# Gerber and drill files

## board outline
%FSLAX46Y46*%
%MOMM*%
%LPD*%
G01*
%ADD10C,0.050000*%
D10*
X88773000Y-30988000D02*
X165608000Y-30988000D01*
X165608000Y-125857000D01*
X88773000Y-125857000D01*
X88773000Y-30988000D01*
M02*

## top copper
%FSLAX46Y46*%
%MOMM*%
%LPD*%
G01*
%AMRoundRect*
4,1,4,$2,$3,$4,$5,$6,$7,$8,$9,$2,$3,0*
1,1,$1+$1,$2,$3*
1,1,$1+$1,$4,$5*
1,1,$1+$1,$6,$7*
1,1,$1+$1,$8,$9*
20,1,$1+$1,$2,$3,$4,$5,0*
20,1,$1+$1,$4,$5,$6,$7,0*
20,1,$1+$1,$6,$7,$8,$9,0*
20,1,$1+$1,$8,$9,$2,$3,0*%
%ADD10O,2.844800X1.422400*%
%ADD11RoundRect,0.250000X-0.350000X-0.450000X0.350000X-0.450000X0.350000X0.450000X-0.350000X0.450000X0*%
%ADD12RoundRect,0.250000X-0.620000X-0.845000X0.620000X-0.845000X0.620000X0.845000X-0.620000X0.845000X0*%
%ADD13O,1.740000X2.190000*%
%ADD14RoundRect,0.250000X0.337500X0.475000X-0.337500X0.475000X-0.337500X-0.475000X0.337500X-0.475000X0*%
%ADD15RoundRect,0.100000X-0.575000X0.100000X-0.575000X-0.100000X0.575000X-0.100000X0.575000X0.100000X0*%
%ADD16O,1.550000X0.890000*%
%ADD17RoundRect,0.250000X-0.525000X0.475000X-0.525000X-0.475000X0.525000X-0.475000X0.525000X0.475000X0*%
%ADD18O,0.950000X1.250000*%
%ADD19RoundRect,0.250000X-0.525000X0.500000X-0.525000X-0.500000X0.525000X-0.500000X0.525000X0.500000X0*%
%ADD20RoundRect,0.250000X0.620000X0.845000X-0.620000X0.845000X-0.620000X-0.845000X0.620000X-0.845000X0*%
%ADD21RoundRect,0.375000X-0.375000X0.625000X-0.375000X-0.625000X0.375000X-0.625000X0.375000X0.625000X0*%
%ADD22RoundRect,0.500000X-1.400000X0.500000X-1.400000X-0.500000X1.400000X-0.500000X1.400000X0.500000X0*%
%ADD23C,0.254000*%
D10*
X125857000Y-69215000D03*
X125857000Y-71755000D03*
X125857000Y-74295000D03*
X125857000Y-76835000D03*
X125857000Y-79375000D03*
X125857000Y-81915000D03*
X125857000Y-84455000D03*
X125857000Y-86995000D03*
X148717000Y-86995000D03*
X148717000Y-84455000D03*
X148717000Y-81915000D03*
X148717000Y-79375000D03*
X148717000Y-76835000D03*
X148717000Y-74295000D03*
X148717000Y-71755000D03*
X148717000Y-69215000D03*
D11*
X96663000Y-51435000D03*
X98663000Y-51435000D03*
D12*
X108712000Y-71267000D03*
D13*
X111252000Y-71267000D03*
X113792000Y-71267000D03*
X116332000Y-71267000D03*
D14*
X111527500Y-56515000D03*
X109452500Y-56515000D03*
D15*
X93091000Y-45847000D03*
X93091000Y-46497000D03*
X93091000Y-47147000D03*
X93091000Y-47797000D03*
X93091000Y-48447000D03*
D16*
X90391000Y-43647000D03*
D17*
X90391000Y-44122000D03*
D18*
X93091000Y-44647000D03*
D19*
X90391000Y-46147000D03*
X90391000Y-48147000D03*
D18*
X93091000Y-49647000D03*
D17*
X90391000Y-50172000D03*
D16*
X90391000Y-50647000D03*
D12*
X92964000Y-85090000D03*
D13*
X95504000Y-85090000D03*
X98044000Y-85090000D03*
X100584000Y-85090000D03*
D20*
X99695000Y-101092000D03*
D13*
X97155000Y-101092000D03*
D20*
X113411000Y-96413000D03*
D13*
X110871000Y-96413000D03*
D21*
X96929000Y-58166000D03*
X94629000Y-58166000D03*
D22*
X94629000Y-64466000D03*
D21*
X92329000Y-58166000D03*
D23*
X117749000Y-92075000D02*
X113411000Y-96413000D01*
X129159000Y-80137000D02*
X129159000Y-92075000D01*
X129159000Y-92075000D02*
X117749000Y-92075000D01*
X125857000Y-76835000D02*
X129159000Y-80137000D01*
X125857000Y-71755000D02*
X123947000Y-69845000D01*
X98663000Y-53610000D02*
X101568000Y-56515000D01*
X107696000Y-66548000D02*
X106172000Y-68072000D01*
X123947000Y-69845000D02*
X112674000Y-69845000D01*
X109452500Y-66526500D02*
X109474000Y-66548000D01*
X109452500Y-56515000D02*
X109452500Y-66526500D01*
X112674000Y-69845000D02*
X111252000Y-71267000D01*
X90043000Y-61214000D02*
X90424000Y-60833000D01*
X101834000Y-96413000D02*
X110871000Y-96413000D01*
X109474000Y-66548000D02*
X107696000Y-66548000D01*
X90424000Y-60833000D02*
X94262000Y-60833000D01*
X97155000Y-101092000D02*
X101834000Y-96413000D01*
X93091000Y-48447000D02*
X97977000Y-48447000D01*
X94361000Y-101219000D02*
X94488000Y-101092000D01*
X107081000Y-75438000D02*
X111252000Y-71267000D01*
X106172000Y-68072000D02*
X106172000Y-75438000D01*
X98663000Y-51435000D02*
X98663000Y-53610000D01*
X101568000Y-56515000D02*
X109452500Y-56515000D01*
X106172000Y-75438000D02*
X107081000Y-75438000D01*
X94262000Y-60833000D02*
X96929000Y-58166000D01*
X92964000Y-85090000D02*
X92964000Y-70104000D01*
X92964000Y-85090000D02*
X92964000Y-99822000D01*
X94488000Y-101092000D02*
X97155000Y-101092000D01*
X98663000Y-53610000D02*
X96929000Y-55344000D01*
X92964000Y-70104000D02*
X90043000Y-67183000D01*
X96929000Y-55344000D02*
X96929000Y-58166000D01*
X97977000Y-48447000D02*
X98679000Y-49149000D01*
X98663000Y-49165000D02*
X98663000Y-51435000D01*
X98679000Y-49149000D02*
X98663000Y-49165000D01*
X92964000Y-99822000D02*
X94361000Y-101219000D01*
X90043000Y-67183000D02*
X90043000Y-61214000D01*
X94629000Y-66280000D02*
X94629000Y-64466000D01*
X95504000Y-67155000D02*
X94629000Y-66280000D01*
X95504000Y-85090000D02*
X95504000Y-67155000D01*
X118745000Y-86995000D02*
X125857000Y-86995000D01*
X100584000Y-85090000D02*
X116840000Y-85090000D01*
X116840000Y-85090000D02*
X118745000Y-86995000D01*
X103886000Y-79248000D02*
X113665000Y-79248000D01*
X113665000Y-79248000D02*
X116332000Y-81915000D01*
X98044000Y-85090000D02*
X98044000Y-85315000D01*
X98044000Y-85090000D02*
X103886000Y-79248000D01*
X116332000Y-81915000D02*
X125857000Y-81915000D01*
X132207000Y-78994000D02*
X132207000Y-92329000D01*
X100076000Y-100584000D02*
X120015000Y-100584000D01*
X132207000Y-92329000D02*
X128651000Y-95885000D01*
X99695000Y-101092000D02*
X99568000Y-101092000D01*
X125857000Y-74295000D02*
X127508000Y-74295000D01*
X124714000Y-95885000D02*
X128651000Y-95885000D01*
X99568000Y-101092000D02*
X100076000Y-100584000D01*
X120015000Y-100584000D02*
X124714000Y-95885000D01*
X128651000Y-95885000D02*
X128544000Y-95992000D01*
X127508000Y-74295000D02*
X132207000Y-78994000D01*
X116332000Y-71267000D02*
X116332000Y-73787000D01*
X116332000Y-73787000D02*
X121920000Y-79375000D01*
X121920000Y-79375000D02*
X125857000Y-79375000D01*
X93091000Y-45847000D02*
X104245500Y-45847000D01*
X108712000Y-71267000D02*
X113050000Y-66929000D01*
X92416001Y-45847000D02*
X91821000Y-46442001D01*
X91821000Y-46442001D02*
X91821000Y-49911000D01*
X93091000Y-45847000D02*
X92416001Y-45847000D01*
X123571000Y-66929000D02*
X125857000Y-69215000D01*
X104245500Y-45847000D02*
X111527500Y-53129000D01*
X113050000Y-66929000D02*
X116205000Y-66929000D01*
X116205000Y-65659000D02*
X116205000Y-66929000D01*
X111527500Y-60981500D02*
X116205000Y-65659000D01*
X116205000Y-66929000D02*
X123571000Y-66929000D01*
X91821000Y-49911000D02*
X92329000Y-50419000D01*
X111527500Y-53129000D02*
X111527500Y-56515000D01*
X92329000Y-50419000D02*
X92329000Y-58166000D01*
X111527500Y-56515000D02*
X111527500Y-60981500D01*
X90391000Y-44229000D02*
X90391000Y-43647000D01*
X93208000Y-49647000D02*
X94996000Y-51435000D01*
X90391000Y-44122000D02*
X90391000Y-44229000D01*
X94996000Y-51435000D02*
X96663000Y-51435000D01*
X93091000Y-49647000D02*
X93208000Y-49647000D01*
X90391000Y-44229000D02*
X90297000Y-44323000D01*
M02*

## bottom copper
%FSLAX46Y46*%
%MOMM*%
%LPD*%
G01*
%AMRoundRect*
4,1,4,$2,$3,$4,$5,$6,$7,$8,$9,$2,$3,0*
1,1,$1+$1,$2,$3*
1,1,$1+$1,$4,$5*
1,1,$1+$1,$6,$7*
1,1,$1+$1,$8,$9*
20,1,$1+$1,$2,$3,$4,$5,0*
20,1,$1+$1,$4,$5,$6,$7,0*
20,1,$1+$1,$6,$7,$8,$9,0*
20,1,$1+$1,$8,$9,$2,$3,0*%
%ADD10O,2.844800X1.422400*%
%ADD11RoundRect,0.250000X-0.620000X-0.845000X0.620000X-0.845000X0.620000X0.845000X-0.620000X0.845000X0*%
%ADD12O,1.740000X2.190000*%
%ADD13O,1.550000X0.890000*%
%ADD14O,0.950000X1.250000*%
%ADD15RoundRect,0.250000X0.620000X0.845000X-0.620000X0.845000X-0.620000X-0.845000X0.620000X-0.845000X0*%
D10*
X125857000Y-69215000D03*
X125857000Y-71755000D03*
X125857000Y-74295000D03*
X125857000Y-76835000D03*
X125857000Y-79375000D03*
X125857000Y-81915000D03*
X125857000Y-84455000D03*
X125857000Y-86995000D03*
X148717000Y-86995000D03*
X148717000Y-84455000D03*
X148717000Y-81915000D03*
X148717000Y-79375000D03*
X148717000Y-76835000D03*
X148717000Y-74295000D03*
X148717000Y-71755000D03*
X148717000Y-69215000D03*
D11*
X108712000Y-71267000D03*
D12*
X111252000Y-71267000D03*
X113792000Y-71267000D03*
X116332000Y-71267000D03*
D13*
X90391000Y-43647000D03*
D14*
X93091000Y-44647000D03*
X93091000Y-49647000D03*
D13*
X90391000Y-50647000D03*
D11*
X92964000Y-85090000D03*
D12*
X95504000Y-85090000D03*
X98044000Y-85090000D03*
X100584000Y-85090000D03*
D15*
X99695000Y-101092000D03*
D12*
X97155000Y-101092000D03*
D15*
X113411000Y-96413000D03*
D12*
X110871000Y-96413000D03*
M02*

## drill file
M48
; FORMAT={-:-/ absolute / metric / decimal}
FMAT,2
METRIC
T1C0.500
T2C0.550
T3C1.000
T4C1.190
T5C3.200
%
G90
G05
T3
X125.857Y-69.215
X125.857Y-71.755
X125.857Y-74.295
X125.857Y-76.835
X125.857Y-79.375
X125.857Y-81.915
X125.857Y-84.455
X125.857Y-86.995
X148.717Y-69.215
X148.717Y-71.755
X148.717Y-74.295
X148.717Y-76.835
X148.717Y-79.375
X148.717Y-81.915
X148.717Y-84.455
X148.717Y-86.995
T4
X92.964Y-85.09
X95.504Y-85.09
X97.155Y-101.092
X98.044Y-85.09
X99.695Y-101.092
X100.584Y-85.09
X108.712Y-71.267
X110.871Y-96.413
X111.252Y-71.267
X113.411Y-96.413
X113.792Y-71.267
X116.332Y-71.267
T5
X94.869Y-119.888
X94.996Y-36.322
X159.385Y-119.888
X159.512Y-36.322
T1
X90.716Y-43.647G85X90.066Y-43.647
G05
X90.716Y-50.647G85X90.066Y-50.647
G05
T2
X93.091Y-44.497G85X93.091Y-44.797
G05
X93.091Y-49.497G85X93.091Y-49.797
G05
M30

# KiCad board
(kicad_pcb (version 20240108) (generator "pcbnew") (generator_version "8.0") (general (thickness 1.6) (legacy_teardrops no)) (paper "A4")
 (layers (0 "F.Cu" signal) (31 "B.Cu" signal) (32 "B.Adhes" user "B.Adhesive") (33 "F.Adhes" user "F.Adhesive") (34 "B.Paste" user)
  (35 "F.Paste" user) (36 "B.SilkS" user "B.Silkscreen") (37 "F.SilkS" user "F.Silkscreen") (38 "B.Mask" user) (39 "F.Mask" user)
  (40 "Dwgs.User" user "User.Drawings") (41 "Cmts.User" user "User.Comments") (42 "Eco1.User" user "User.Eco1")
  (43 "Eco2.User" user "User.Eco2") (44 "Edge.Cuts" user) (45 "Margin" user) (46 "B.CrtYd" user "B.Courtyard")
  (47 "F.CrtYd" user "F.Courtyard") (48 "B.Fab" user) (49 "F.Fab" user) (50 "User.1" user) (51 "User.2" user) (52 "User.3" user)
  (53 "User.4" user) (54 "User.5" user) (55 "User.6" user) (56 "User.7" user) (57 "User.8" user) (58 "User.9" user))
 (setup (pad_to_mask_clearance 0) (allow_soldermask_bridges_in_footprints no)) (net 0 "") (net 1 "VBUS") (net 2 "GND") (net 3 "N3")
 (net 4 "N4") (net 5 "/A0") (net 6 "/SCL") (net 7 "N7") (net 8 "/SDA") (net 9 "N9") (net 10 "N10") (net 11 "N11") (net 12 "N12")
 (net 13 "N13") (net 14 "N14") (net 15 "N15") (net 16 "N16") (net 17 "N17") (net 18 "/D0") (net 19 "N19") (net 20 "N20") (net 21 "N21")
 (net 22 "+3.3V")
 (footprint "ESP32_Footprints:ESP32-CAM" (layer "F.Cu") (at 137.287 79.375)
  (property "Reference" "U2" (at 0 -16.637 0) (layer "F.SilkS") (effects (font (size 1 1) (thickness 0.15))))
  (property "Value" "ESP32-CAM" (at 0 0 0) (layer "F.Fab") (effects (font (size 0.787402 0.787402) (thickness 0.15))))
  (pad "P$1" thru_hole oval (at -11.43 -10.16) (size 2.8448 1.4224) (drill 1) (layers "*.Cu" "*.Mask") (remove_unused_layers no)
   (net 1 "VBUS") (solder_mask_margin 0.102))
  (pad "P$2" thru_hole oval (at -11.43 -7.62) (size 2.8448 1.4224) (drill 1) (layers "*.Cu" "*.Mask") (remove_unused_layers no)
   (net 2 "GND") (solder_mask_margin 0.102))
  (pad "P$3" thru_hole oval (at -11.43 -5.08) (size 2.8448 1.4224) (drill 1) (layers "*.Cu" "*.Mask") (remove_unused_layers no) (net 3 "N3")
   (solder_mask_margin 0.102))
  (pad "P$4" thru_hole oval (at -11.43 -2.54) (size 2.8448 1.4224) (drill 1) (layers "*.Cu" "*.Mask") (remove_unused_layers no) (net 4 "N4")
   (solder_mask_margin 0.102))
  (pad "P$5" thru_hole oval (at -11.43 0) (size 2.8448 1.4224) (drill 1) (layers "*.Cu" "*.Mask") (remove_unused_layers no) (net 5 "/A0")
   (solder_mask_margin 0.102))
  (pad "P$6" thru_hole oval (at -11.43 2.54) (size 2.8448 1.4224) (drill 1) (layers "*.Cu" "*.Mask") (remove_unused_layers no)
   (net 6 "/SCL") (solder_mask_margin 0.102))
  (pad "P$7" thru_hole oval (at -11.43 5.08) (size 2.8448 1.4224) (drill 1) (layers "*.Cu" "*.Mask") (remove_unused_layers no) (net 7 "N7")
   (solder_mask_margin 0.102))
  (pad "P$8" thru_hole oval (at -11.43 7.62) (size 2.8448 1.4224) (drill 1) (layers "*.Cu" "*.Mask") (remove_unused_layers no)
   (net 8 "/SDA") (solder_mask_margin 0.102))
  (pad "P$9" thru_hole oval (at 11.43 7.62) (size 2.8448 1.4224) (drill 1) (layers "*.Cu" "*.Mask") (remove_unused_layers no) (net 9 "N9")
   (solder_mask_margin 0.102))
  (pad "P$10" thru_hole oval (at 11.43 5.08) (size 2.8448 1.4224) (drill 1) (layers "*.Cu" "*.Mask") (remove_unused_layers no)
   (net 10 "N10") (solder_mask_margin 0.102))
  (pad "P$11" thru_hole oval (at 11.43 2.54) (size 2.8448 1.4224) (drill 1) (layers "*.Cu" "*.Mask") (remove_unused_layers no)
   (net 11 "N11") (solder_mask_margin 0.102))
  (pad "P$12" thru_hole oval (at 11.43 0) (size 2.8448 1.4224) (drill 1) (layers "*.Cu" "*.Mask") (remove_unused_layers no) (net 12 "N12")
   (solder_mask_margin 0.102))
  (pad "P$13" thru_hole oval (at 11.43 -2.54) (size 2.8448 1.4224) (drill 1) (layers "*.Cu" "*.Mask") (remove_unused_layers no)
   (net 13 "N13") (solder_mask_margin 0.102))
  (pad "P$14" thru_hole oval (at 11.43 -5.08) (size 2.8448 1.4224) (drill 1) (layers "*.Cu" "*.Mask") (remove_unused_layers no)
   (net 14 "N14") (solder_mask_margin 0.102))
  (pad "P$15" thru_hole oval (at 11.43 -7.62) (size 2.8448 1.4224) (drill 1) (layers "*.Cu" "*.Mask") (remove_unused_layers no)
   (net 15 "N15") (solder_mask_margin 0.102))
  (pad "P$16" thru_hole oval (at 11.43 -10.16) (size 2.8448 1.4224) (drill 1) (layers "*.Cu" "*.Mask") (remove_unused_layers no)
   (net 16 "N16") (solder_mask_margin 0.102)))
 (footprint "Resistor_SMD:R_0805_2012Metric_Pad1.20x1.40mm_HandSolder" (layer "F.Cu") (at 97.663 51.435)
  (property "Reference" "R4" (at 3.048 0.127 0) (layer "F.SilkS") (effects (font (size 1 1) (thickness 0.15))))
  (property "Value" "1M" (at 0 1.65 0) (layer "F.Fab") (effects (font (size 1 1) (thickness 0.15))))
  (pad "1" smd roundrect (at -1 0) (size 1.2 1.4) (layers "F.Cu" "F.Paste" "F.Mask") (roundrect_rratio 0.208333) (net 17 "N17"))
  (pad "2" smd roundrect (at 1 0) (size 1.2 1.4) (layers "F.Cu" "F.Paste" "F.Mask") (roundrect_rratio 0.208333) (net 2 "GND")))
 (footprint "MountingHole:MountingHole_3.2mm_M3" (layer "F.Cu") (at 159.512 36.322)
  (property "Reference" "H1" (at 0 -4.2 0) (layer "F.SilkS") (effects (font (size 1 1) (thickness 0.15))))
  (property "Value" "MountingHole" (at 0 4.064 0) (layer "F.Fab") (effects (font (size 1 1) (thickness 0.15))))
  (pad "" np_thru_hole circle (at 0 0) (size 3.2 3.2) (drill 3.2) (layers "*.Cu" "*.Mask")))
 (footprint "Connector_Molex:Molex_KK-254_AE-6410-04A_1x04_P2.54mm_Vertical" (layer "F.Cu") (at 108.712 71.267)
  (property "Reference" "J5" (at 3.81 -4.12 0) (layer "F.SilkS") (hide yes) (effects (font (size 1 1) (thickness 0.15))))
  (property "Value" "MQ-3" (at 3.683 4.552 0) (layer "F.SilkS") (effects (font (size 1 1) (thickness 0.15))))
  (pad "1" thru_hole roundrect (at 0 0) (size 1.74 2.19) (drill 1.19) (layers "*.Cu" "*.Mask") (remove_unused_layers no)
   (roundrect_rratio 0.143678) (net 1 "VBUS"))
  (pad "2" thru_hole oval (at 2.54 0) (size 1.74 2.19) (drill 1.19) (layers "*.Cu" "*.Mask") (remove_unused_layers no) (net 2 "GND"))
  (pad "3" thru_hole oval (at 5.08 0) (size 1.74 2.19) (drill 1.19) (layers "*.Cu" "*.Mask") (remove_unused_layers no) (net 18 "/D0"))
  (pad "4" thru_hole oval (at 7.62 0) (size 1.74 2.19) (drill 1.19) (layers "*.Cu" "*.Mask") (remove_unused_layers no) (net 5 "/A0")))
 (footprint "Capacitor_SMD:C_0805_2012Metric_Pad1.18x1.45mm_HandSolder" (layer "F.Cu") (at 110.49 56.515 180)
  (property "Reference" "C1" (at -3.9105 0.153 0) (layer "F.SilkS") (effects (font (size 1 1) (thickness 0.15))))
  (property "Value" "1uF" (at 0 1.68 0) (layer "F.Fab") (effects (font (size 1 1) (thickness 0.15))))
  (pad "1" smd roundrect (at -1.0375 0 180) (size 1.175 1.45) (layers "F.Cu" "F.Paste" "F.Mask") (roundrect_rratio 0.212766) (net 1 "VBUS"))
  (pad "2" smd roundrect (at 1.0375 0 180) (size 1.175 1.45) (layers "F.Cu" "F.Paste" "F.Mask") (roundrect_rratio 0.212766) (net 2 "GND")))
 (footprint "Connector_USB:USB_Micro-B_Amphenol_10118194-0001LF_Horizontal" (layer "F.Cu") (at 91.691 47.147 -90)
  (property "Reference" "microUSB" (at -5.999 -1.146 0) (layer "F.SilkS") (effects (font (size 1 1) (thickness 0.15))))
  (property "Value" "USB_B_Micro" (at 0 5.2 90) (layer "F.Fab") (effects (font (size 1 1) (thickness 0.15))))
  (pad "" smd oval (at -3.5 1.3 270) (size 0.89 1.55) (layers "F.Paste"))
  (pad "" smd oval (at -2.5 -1.4 270) (size 1.25 0.95) (layers "F.Paste"))
  (pad "" smd oval (at 2.5 -1.4 270) (size 1.25 0.95) (layers "F.Paste"))
  (pad "" smd oval (at 3.5 1.3 270) (size 0.89 1.55) (layers "F.Paste"))
  (pad "1" smd roundrect (at -1.3 -1.4 270) (size 0.4 1.35) (layers "F.Cu" "F.Paste" "F.Mask") (roundrect_rratio 0.25) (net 1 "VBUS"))
  (pad "2" smd roundrect (at -0.65 -1.4 270) (size 0.4 1.35) (layers "F.Cu" "F.Paste" "F.Mask") (roundrect_rratio 0.25) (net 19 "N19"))
  (pad "3" smd roundrect (at 0 -1.4 270) (size 0.4 1.35) (layers "F.Cu" "F.Paste" "F.Mask") (roundrect_rratio 0.25) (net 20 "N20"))
  (pad "4" smd roundrect (at 0.65 -1.4 270) (size 0.4 1.35) (layers "F.Cu" "F.Paste" "F.Mask") (roundrect_rratio 0.25) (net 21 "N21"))
  (pad "5" smd roundrect (at 1.3 -1.4 270) (size 0.4 1.35) (layers "F.Cu" "F.Paste" "F.Mask") (roundrect_rratio 0.25) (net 2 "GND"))
  (pad "6" thru_hole oval (at -3.5 1.3 270) (size 0.89 1.55) (drill oval 0.5 1.15) (layers "*.Cu" "*.Mask") (remove_unused_layers no)
   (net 17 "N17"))
  (pad "6" smd roundrect (at -3.025 1.3 270) (size 1.45 1.55) (layers "F.Cu" "F.Paste" "F.Mask") (roundrect_rratio 0.1724137931)
   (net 17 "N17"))
  (pad "6" thru_hole oval (at -2.5 -1.4 270) (size 1.25 0.95) (drill oval 0.85 0.55) (layers "*.Cu" "*.Mask") (remove_unused_layers no)
   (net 17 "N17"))
  (pad "6" smd roundrect (at -1 1.3 270) (size 1.5 1.55) (layers "F.Cu" "F.Paste" "F.Mask") (roundrect_rratio 0.1666666667) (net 17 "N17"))
  (pad "6" smd roundrect (at 1 1.3 270) (size 1.5 1.55) (layers "F.Cu" "F.Paste" "F.Mask") (roundrect_rratio 0.1666666667) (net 17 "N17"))
  (pad "6" thru_hole oval (at 2.5 -1.4 270) (size 1.25 0.95) (drill oval 0.85 0.55) (layers "*.Cu" "*.Mask") (remove_unused_layers no)
   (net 17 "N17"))
  (pad "6" smd roundrect (at 3.025 1.3 270) (size 1.45 1.55) (layers "F.Cu" "F.Paste" "F.Mask") (roundrect_rratio 0.1724137931)
   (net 17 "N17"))
  (pad "6" thru_hole oval (at 3.5 1.3 270) (size 0.89 1.55) (drill oval 0.5 1.15) (layers "*.Cu" "*.Mask") (remove_unused_layers no)
   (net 17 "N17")))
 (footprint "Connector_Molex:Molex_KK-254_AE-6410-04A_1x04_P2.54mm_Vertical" (layer "F.Cu") (at 92.964 85.09)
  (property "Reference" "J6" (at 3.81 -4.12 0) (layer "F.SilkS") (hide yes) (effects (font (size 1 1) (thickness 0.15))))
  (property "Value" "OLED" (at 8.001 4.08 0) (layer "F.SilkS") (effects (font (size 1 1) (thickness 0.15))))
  (pad "1" thru_hole roundrect (at 0 0) (size 1.74 2.19) (drill 1.19) (layers "*.Cu" "*.Mask") (remove_unused_layers no)
   (roundrect_rratio 0.143678) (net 2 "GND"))
  (pad "2" thru_hole oval (at 2.54 0) (size 1.74 2.19) (drill 1.19) (layers "*.Cu" "*.Mask") (remove_unused_layers no) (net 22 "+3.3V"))
  (pad "3" thru_hole oval (at 5.08 0) (size 1.74 2.19) (drill 1.19) (layers "*.Cu" "*.Mask") (remove_unused_layers no) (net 6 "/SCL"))
  (pad "4" thru_hole oval (at 7.62 0) (size 1.74 2.19) (drill 1.19) (layers "*.Cu" "*.Mask") (remove_unused_layers no) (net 8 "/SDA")))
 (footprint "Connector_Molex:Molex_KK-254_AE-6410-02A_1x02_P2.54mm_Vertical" (layer "F.Cu") (at 99.695 101.092 180)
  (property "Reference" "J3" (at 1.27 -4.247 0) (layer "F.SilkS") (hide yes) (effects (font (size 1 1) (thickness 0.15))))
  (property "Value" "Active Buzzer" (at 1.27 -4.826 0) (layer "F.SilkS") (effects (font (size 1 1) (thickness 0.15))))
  (pad "1" thru_hole roundrect (at 0 0 180) (size 1.74 2.19) (drill 1.19) (layers "*.Cu" "*.Mask") (remove_unused_layers no)
   (roundrect_rratio 0.143678) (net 3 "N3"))
  (pad "2" thru_hole oval (at 2.54 0 180) (size 1.74 2.19) (drill 1.19) (layers "*.Cu" "*.Mask") (remove_unused_layers no) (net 2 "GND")))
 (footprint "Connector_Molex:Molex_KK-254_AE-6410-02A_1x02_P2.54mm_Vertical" (layer "F.Cu") (at 113.411 96.413 180)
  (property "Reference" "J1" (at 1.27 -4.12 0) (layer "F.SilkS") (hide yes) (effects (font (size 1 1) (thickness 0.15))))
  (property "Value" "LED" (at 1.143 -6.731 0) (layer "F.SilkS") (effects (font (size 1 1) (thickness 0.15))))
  (pad "1" thru_hole roundrect (at 0 0 180) (size 1.74 2.19) (drill 1.19) (layers "*.Cu" "*.Mask") (remove_unused_layers no)
   (roundrect_rratio 0.143678) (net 4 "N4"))
  (pad "2" thru_hole oval (at 2.54 0 180) (size 1.74 2.19) (drill 1.19) (layers "*.Cu" "*.Mask") (remove_unused_layers no) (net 2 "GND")))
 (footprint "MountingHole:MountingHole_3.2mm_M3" (layer "F.Cu") (at 94.869 119.888)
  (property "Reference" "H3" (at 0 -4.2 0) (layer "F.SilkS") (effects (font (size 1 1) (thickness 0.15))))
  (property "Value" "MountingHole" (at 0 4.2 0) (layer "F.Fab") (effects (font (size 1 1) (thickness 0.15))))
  (pad "" np_thru_hole circle (at 0 0) (size 3.2 3.2) (drill 3.2) (layers "*.Cu" "*.Mask")))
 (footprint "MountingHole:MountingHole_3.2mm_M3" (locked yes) (layer "F.Cu") (at 159.385 119.888)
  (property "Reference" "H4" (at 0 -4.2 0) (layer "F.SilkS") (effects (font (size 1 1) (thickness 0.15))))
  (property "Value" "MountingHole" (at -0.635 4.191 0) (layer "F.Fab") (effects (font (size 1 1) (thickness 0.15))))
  (pad "" np_thru_hole circle (at 0 0) (size 3.2 3.2) (drill 3.2) (layers "*.Cu" "*.Mask")))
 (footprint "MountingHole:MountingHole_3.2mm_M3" (layer "F.Cu") (at 94.996 36.322)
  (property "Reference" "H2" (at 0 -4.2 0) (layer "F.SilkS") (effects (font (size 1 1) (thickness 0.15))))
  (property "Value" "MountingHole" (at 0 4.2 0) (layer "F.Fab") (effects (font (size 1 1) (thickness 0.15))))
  (pad "" np_thru_hole circle (at 0 0) (size 3.2 3.2) (drill 3.2) (layers "*.Cu" "*.Mask")))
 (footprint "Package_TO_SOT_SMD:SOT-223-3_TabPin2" (layer "F.Cu") (at 94.629 61.316 -90)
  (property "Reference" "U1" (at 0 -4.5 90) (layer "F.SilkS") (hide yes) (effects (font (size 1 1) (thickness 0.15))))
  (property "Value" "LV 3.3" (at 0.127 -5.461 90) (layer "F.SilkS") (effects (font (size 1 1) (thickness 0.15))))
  (pad "1" smd roundrect (at -3.15 -2.3 270) (size 2 1.5) (layers "F.Cu" "F.Paste" "F.Mask") (roundrect_rratio 0.25) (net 2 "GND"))
  (pad "2" smd roundrect (at -3.15 0 270) (size 2 1.5) (layers "F.Cu" "F.Paste" "F.Mask") (roundrect_rratio 0.25) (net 22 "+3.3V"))
  (pad "2" smd roundrect (at 3.15 0 270) (size 2 3.8) (layers "F.Cu" "F.Paste" "F.Mask") (roundrect_rratio 0.25) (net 22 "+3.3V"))
  (pad "3" smd roundrect (at -3.15 2.3 270) (size 2 1.5) (layers "F.Cu" "F.Paste" "F.Mask") (roundrect_rratio 0.25) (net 1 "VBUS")))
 (gr_rect (start 88.773 30.988) (end 165.608 125.857) (locked yes) (stroke (width 0.05) (type default)) (fill none) (layer "Edge.Cuts"))
 (segment (start 117.749 92.075) (end 113.411 96.413) (width 0.254) (layer "F.Cu") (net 4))
 (segment (start 129.159 80.137) (end 129.159 92.075) (width 0.254) (layer "F.Cu") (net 4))
 (segment (start 129.159 92.075) (end 117.749 92.075) (width 0.254) (layer "F.Cu") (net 4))
 (segment (start 125.857 76.835) (end 129.159 80.137) (width 0.254) (layer "F.Cu") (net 4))
 (segment (start 125.857 71.755) (end 123.947 69.845) (width 0.254) (layer "F.Cu") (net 2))
 (segment (start 98.663 53.61) (end 101.568 56.515) (width 0.254) (layer "F.Cu") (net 2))
 (segment (start 107.696 66.548) (end 106.172 68.072) (width 0.254) (layer "F.Cu") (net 2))
 (segment (start 123.947 69.845) (end 112.674 69.845) (width 0.254) (layer "F.Cu") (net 2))
 (segment (start 109.4525 66.5265) (end 109.474 66.548) (width 0.254) (layer "F.Cu") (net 2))
 (segment (start 109.4525 56.515) (end 109.4525 66.5265) (width 0.254) (layer "F.Cu") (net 2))
 (segment (start 112.674 69.845) (end 111.252 71.267) (width 0.254) (layer "F.Cu") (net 2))
 (segment (start 90.043 61.214) (end 90.424 60.833) (width 0.254) (layer "F.Cu") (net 2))
 (segment (start 101.834 96.413) (end 110.871 96.413) (width 0.254) (layer "F.Cu") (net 2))
 (segment (start 109.474 66.548) (end 107.696 66.548) (width 0.254) (layer "F.Cu") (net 2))
 (segment (start 90.424 60.833) (end 94.262 60.833) (width 0.254) (layer "F.Cu") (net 2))
 (segment (start 97.155 101.092) (end 101.834 96.413) (width 0.254) (layer "F.Cu") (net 2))
 (segment (start 93.091 48.447) (end 97.977 48.447) (width 0.254) (layer "F.Cu") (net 2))
 (segment (start 94.361 101.219) (end 94.488 101.092) (width 0.254) (layer "F.Cu") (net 2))
 (segment (start 107.081 75.438) (end 111.252 71.267) (width 0.254) (layer "F.Cu") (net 2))
 (segment (start 106.172 68.072) (end 106.172 75.438) (width 0.254) (layer "F.Cu") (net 2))
 (segment (start 98.663 51.435) (end 98.663 53.61) (width 0.254) (layer "F.Cu") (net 2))
 (segment (start 101.568 56.515) (end 109.4525 56.515) (width 0.254) (layer "F.Cu") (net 2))
 (segment (start 106.172 75.438) (end 107.081 75.438) (width 0.254) (layer "F.Cu") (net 2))
 (segment (start 94.262 60.833) (end 96.929 58.166) (width 0.254) (layer "F.Cu") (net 2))
 (segment (start 92.964 85.09) (end 92.964 70.104) (width 0.254) (layer "F.Cu") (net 2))
 (segment (start 92.964 85.09) (end 92.964 99.822) (width 0.254) (layer "F.Cu") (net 2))
 (segment (start 94.488 101.092) (end 97.155 101.092) (width 0.254) (layer "F.Cu") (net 2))
 (segment (start 98.663 53.61) (end 96.929 55.344) (width 0.254) (layer "F.Cu") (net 2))
 (segment (start 92.964 70.104) (end 90.043 67.183) (width 0.254) (layer "F.Cu") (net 2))
 (segment (start 96.929 55.344) (end 96.929 58.166) (width 0.254) (layer "F.Cu") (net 2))
 (segment (start 97.977 48.447) (end 98.679 49.149) (width 0.254) (layer "F.Cu") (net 2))
 (segment (start 98.663 49.165) (end 98.663 51.435) (width 0.254) (layer "F.Cu") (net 2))
 (segment (start 98.679 49.149) (end 98.663 49.165) (width 0.254) (layer "F.Cu") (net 2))
 (segment (start 92.964 99.822) (end 94.361 101.219) (width 0.254) (layer "F.Cu") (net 2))
 (segment (start 90.043 67.183) (end 90.043 61.214) (width 0.254) (layer "F.Cu") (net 2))
 (segment (start 94.629 66.28) (end 94.629 64.466) (width 0.254) (layer "F.Cu") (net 22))
 (segment (start 95.504 67.155) (end 94.629 66.28) (width 0.254) (layer "F.Cu") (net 22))
 (segment (start 95.504 85.09) (end 95.504 67.155) (width 0.254) (layer "F.Cu") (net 22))
 (segment (start 118.745 86.995) (end 125.857 86.995) (width 0.254) (layer "F.Cu") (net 8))
 (segment (start 100.584 85.09) (end 116.84 85.09) (width 0.254) (layer "F.Cu") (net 8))
 (segment (start 116.84 85.09) (end 118.745 86.995) (width 0.254) (layer "F.Cu") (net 8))
 (segment (start 103.886 79.248) (end 113.665 79.248) (width 0.254) (layer "F.Cu") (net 6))
 (segment (start 113.665 79.248) (end 116.332 81.915) (width 0.254) (layer "F.Cu") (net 6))
 (segment (start 98.044 85.09) (end 98.044 85.315) (width 0.254) (layer "F.Cu") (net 6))
 (segment (start 98.044 85.09) (end 103.886 79.248) (width 0.254) (layer "F.Cu") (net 6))
 (segment (start 116.332 81.915) (end 125.857 81.915) (width 0.254) (layer "F.Cu") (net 6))
 (segment (start 132.207 78.994) (end 132.207 92.329) (width 0.254) (layer "F.Cu") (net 3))
 (segment (start 100.076 100.584) (end 120.015 100.584) (width 0.254) (layer "F.Cu") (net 3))
 (segment (start 132.207 92.329) (end 128.651 95.885) (width 0.254) (layer "F.Cu") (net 3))
 (segment (start 99.695 101.092) (end 99.568 101.092) (width 0.254) (layer "F.Cu") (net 3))
 (segment (start 125.857 74.295) (end 127.508 74.295) (width 0.254) (layer "F.Cu") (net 3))
 (segment (start 124.714 95.885) (end 128.651 95.885) (width 0.254) (layer "F.Cu") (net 3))
 (segment (start 99.568 101.092) (end 100.076 100.584) (width 0.254) (layer "F.Cu") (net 3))
 (segment (start 120.015 100.584) (end 124.714 95.885) (width 0.254) (layer "F.Cu") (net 3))
 (segment (start 128.651 95.885) (end 128.544 95.992) (width 0.254) (layer "F.Cu") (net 3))
 (segment (start 127.508 74.295) (end 132.207 78.994) (width 0.254) (layer "F.Cu") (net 3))
 (segment (start 116.332 71.267) (end 116.332 73.787) (width 0.254) (layer "F.Cu") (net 5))
 (segment (start 116.332 73.787) (end 121.92 79.375) (width 0.254) (layer "F.Cu") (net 5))
 (segment (start 121.92 79.375) (end 125.857 79.375) (width 0.254) (layer "F.Cu") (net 5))
 (segment (start 93.091 45.847) (end 104.2455 45.847) (width 0.254) (layer "F.Cu") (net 1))
 (segment (start 108.712 71.267) (end 113.05 66.929) (width 0.254) (layer "F.Cu") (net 1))
 (segment (start 92.416001 45.847) (end 91.821 46.442001) (width 0.254) (layer "F.Cu") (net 1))
 (segment (start 91.821 46.442001) (end 91.821 49.911) (width 0.254) (layer "F.Cu") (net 1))
 (segment (start 93.091 45.847) (end 92.416001 45.847) (width 0.254) (layer "F.Cu") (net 1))
 (segment (start 123.571 66.929) (end 125.857 69.215) (width 0.254) (layer "F.Cu") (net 1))
 (segment (start 104.2455 45.847) (end 111.5275 53.129) (width 0.254) (layer "F.Cu") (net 1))
 (segment (start 113.05 66.929) (end 116.205 66.929) (width 0.254) (layer "F.Cu") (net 1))
 (segment (start 116.205 65.659) (end 116.205 66.929) (width 0.254) (layer "F.Cu") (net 1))
 (segment (start 111.5275 60.9815) (end 116.205 65.659) (width 0.254) (layer "F.Cu") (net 1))
 (segment (start 116.205 66.929) (end 123.571 66.929) (width 0.254) (layer "F.Cu") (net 1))
 (segment (start 91.821 49.911) (end 92.329 50.419) (width 0.254) (layer "F.Cu") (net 1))
 (segment (start 111.5275 53.129) (end 111.5275 56.515) (width 0.254) (layer "F.Cu") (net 1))
 (segment (start 92.329 50.419) (end 92.329 58.166) (width 0.254) (layer "F.Cu") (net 1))
 (segment (start 111.5275 56.515) (end 111.5275 60.9815) (width 0.254) (layer "F.Cu") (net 1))
 (segment (start 90.391 44.229) (end 90.391 43.647) (width 0.254) (layer "F.Cu") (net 17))
 (segment (start 93.208 49.647) (end 94.996 51.435) (width 0.254) (layer "F.Cu") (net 17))
 (segment (start 90.391 44.122) (end 90.391 44.229) (width 0.254) (layer "F.Cu") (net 17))
 (segment (start 94.996 51.435) (end 96.663 51.435) (width 0.254) (layer "F.Cu") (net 17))
 (segment (start 93.091 49.647) (end 93.208 49.647) (width 0.254) (layer "F.Cu") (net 17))
 (segment (start 90.391 44.229) (end 90.297 44.323) (width 0.254) (layer "F.Cu") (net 17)))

